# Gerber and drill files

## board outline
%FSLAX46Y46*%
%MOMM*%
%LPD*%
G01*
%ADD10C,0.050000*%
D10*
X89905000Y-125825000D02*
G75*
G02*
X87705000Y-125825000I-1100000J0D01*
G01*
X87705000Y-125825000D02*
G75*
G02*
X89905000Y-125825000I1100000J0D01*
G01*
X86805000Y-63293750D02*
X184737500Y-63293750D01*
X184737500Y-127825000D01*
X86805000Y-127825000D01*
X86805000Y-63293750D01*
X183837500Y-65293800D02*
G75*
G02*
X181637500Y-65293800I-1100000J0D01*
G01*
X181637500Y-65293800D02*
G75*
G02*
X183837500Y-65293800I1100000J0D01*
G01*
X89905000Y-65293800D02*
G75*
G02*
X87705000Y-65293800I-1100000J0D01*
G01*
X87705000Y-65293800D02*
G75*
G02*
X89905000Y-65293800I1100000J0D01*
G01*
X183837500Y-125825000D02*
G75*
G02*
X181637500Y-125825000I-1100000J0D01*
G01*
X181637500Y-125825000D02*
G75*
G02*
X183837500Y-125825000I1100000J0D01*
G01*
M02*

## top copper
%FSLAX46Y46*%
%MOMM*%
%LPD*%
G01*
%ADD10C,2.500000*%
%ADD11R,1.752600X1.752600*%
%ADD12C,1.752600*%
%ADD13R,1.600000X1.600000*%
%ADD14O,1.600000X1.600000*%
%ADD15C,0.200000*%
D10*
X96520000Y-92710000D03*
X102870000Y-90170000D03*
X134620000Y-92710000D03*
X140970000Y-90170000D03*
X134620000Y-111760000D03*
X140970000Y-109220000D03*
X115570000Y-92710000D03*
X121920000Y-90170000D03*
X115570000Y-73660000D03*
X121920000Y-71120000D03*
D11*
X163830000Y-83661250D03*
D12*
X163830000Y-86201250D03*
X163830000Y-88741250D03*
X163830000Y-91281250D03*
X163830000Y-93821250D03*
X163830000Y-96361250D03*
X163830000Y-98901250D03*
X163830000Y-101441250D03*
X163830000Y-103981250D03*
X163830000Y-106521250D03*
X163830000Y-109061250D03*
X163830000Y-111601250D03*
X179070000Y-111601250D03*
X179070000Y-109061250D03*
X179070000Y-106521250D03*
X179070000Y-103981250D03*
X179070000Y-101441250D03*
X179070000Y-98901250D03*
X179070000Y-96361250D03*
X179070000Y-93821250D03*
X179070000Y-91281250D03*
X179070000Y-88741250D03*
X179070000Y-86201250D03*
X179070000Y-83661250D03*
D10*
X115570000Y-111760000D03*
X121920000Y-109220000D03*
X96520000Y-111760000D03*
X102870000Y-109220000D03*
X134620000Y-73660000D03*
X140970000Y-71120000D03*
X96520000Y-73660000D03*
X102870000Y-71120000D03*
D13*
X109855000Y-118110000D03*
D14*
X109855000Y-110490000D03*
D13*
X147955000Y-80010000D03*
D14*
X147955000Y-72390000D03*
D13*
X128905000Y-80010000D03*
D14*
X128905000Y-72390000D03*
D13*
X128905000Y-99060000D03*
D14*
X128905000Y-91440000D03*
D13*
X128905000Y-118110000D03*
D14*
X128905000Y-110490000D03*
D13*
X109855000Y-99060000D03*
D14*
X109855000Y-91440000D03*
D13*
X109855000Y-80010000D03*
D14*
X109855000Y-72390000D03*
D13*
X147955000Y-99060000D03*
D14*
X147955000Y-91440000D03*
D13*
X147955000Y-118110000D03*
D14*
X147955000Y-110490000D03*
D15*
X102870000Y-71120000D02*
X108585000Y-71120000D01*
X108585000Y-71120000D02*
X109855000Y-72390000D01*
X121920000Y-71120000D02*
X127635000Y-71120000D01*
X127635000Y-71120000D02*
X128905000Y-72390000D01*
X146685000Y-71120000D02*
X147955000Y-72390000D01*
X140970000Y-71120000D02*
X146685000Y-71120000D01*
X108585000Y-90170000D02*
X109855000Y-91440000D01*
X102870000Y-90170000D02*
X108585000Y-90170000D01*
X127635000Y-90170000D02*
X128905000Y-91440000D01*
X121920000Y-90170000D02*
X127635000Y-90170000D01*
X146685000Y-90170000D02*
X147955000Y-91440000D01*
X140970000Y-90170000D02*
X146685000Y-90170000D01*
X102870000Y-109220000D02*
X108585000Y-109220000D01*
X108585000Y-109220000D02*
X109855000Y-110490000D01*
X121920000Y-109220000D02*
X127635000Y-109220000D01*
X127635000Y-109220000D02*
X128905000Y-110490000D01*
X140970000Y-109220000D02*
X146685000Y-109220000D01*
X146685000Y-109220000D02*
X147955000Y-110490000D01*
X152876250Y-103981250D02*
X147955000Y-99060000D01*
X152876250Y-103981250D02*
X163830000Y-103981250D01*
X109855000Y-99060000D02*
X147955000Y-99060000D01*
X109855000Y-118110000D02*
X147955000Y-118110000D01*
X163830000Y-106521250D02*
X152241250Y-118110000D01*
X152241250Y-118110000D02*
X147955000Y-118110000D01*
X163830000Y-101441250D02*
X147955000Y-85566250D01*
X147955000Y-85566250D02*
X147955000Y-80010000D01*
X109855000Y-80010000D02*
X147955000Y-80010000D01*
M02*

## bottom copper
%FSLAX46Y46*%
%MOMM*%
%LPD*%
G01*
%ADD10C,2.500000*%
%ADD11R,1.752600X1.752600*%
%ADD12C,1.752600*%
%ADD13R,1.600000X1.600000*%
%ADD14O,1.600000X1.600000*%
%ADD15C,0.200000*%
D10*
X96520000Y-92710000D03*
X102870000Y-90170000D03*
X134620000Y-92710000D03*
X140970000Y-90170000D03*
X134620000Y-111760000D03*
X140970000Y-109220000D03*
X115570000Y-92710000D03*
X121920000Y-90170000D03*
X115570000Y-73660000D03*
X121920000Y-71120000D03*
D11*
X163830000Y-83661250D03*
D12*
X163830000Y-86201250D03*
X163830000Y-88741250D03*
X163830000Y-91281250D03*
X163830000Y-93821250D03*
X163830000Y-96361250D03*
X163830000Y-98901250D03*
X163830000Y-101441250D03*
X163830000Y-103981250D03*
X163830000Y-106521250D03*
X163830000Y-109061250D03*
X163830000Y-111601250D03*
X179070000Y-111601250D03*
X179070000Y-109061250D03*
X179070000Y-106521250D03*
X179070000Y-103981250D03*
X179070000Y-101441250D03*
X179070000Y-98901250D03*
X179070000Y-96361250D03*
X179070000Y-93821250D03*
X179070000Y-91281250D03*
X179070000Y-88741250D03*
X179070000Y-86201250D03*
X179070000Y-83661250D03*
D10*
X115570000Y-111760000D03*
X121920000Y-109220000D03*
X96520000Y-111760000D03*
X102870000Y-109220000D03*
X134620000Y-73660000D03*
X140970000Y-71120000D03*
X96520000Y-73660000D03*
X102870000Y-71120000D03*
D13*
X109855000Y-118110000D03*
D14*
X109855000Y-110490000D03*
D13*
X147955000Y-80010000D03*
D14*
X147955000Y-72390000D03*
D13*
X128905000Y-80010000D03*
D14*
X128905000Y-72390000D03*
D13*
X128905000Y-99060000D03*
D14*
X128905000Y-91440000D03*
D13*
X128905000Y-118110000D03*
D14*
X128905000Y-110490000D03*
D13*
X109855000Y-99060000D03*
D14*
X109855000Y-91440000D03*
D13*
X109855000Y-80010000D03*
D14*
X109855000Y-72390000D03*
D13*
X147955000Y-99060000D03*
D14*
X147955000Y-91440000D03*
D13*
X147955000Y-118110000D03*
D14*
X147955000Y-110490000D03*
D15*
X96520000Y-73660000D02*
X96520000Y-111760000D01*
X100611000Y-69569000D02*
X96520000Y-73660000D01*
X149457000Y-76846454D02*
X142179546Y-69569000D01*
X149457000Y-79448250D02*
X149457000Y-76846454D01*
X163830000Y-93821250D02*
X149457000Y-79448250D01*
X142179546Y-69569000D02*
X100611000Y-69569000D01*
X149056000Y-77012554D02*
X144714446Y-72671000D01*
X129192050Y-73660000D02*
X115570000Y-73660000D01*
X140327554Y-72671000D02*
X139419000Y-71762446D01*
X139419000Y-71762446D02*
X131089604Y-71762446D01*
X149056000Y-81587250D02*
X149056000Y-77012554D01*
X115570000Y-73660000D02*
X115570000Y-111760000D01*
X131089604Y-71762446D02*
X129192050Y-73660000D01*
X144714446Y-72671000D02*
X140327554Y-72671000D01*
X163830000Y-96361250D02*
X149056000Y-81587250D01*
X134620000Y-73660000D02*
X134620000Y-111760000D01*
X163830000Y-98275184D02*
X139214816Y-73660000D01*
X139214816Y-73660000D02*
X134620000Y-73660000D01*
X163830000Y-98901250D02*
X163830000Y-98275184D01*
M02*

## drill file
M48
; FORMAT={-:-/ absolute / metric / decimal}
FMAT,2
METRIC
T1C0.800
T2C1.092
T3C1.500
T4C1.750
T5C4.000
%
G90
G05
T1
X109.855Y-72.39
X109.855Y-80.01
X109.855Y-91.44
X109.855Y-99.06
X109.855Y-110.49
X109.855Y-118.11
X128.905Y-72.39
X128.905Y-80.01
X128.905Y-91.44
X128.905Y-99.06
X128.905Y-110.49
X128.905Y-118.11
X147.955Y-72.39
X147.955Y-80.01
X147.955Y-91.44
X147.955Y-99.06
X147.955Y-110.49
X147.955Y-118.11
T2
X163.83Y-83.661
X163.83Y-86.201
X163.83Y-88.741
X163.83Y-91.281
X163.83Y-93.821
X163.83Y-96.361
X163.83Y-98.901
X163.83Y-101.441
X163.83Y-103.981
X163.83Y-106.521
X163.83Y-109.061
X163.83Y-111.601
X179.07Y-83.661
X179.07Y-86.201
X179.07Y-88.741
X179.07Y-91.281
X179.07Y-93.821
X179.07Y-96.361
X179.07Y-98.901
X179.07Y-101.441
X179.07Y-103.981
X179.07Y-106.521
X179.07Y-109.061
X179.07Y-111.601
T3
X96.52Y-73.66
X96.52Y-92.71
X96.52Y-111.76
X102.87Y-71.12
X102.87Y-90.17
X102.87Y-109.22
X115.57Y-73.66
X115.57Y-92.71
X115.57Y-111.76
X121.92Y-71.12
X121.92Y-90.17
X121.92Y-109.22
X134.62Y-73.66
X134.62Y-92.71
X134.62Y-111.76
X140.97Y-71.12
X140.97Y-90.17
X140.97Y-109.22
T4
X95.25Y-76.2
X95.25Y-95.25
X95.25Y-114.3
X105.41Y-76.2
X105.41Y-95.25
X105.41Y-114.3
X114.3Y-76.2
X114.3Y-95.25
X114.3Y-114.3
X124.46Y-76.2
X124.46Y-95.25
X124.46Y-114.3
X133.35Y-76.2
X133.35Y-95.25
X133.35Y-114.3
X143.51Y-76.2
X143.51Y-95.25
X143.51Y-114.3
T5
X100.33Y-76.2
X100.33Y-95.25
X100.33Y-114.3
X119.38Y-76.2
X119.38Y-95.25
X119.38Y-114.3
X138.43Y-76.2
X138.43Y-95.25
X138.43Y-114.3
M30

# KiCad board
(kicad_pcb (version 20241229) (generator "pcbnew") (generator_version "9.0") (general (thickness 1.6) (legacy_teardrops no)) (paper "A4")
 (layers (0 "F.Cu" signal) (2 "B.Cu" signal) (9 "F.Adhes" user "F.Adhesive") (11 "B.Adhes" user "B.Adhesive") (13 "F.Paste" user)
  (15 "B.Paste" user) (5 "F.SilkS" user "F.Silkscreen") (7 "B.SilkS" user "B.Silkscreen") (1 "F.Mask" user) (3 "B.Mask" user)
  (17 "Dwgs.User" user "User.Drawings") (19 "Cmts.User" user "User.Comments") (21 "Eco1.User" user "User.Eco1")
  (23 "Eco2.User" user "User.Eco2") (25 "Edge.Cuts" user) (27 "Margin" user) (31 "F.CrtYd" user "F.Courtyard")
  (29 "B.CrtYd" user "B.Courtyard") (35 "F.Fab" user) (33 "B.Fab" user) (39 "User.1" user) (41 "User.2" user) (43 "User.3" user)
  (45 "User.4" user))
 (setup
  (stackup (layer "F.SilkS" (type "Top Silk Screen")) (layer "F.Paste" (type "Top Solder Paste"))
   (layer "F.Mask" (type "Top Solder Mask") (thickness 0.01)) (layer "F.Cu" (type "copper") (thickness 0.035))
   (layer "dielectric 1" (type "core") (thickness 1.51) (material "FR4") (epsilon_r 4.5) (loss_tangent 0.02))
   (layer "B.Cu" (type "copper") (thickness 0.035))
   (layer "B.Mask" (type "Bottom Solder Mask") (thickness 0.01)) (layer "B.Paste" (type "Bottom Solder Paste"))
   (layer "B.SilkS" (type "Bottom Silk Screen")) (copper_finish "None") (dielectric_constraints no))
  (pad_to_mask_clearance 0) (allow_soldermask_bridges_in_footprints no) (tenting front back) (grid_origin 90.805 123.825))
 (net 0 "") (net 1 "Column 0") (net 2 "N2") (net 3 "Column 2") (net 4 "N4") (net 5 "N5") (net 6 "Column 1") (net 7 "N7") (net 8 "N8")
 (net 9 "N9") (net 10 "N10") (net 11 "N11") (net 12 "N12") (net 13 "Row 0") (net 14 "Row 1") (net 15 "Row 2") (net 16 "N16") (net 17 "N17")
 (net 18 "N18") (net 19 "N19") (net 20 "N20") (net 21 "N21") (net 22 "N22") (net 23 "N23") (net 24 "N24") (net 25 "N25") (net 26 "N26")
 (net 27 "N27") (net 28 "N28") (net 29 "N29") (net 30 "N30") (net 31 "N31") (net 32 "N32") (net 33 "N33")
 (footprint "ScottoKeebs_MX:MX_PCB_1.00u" (layer "F.Cu") (at 100.33 95.25)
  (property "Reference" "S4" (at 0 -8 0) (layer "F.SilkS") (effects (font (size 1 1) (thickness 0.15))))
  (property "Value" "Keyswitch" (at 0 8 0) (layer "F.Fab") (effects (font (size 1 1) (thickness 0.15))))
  (pad "" np_thru_hole circle (at -5.08 0) (size 1.75 1.75) (drill 1.75) (layers "*.Cu" "*.Mask"))
  (pad "" np_thru_hole circle (at 0 0) (size 4 4) (drill 4) (layers "*.Cu" "*.Mask"))
  (pad "" np_thru_hole circle (at 5.08 0) (size 1.75 1.75) (drill 1.75) (layers "*.Cu" "*.Mask"))
  (pad "1" thru_hole circle (at -3.81 -2.54) (size 2.5 2.5) (drill 1.5) (layers "*.Cu" "*.Mask") (remove_unused_layers no)
   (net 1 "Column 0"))
  (pad "2" thru_hole circle (at 2.54 -5.08) (size 2.5 2.5) (drill 1.5) (layers "*.Cu" "*.Mask") (remove_unused_layers no) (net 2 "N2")))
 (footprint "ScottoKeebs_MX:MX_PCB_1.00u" (layer "F.Cu") (at 138.43 95.25)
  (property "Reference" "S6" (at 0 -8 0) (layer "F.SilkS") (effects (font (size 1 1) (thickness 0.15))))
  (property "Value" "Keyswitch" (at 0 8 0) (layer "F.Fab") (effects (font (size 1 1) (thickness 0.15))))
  (pad "" np_thru_hole circle (at -5.08 0) (size 1.75 1.75) (drill 1.75) (layers "*.Cu" "*.Mask"))
  (pad "" np_thru_hole circle (at 0 0) (size 4 4) (drill 4) (layers "*.Cu" "*.Mask"))
  (pad "" np_thru_hole circle (at 5.08 0) (size 1.75 1.75) (drill 1.75) (layers "*.Cu" "*.Mask"))
  (pad "1" thru_hole circle (at -3.81 -2.54) (size 2.5 2.5) (drill 1.5) (layers "*.Cu" "*.Mask") (remove_unused_layers no)
   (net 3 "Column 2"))
  (pad "2" thru_hole circle (at 2.54 -5.08) (size 2.5 2.5) (drill 1.5) (layers "*.Cu" "*.Mask") (remove_unused_layers no) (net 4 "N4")))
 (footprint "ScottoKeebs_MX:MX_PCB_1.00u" (layer "F.Cu") (at 138.43 114.3)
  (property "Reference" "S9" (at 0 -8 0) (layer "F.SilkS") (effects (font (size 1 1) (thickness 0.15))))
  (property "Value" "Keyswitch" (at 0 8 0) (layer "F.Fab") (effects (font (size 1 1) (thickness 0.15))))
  (pad "" np_thru_hole circle (at -5.08 0) (size 1.75 1.75) (drill 1.75) (layers "*.Cu" "*.Mask"))
  (pad "" np_thru_hole circle (at 0 0) (size 4 4) (drill 4) (layers "*.Cu" "*.Mask"))
  (pad "" np_thru_hole circle (at 5.08 0) (size 1.75 1.75) (drill 1.75) (layers "*.Cu" "*.Mask"))
  (pad "1" thru_hole circle (at -3.81 -2.54) (size 2.5 2.5) (drill 1.5) (layers "*.Cu" "*.Mask") (remove_unused_layers no)
   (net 3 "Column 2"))
  (pad "2" thru_hole circle (at 2.54 -5.08) (size 2.5 2.5) (drill 1.5) (layers "*.Cu" "*.Mask") (remove_unused_layers no) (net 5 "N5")))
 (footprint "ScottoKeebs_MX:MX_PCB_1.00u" (layer "F.Cu") (at 119.38 95.25)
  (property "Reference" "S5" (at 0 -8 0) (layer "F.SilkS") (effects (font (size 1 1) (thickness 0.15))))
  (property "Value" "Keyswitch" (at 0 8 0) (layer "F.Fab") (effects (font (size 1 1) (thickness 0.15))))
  (pad "" np_thru_hole circle (at -5.08 0) (size 1.75 1.75) (drill 1.75) (layers "*.Cu" "*.Mask"))
  (pad "" np_thru_hole circle (at 0 0) (size 4 4) (drill 4) (layers "*.Cu" "*.Mask"))
  (pad "" np_thru_hole circle (at 5.08 0) (size 1.75 1.75) (drill 1.75) (layers "*.Cu" "*.Mask"))
  (pad "1" thru_hole circle (at -3.81 -2.54) (size 2.5 2.5) (drill 1.5) (layers "*.Cu" "*.Mask") (remove_unused_layers no)
   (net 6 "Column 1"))
  (pad "2" thru_hole circle (at 2.54 -5.08) (size 2.5 2.5) (drill 1.5) (layers "*.Cu" "*.Mask") (remove_unused_layers no) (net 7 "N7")))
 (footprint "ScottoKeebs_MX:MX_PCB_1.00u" (layer "F.Cu") (at 119.38 76.2)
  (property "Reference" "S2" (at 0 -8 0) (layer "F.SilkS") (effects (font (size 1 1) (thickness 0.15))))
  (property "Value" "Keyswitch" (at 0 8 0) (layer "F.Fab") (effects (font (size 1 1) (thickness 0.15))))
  (pad "" np_thru_hole circle (at -5.08 0) (size 1.75 1.75) (drill 1.75) (layers "*.Cu" "*.Mask"))
  (pad "" np_thru_hole circle (at 0 0) (size 4 4) (drill 4) (layers "*.Cu" "*.Mask"))
  (pad "" np_thru_hole circle (at 5.08 0) (size 1.75 1.75) (drill 1.75) (layers "*.Cu" "*.Mask"))
  (pad "1" thru_hole circle (at -3.81 -2.54) (size 2.5 2.5) (drill 1.5) (layers "*.Cu" "*.Mask") (remove_unused_layers no)
   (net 6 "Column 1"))
  (pad "2" thru_hole circle (at 2.54 -5.08) (size 2.5 2.5) (drill 1.5) (layers "*.Cu" "*.Mask") (remove_unused_layers no) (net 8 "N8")))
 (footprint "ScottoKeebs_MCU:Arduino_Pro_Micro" (layer "F.Cu") (at 171.45 97.63125)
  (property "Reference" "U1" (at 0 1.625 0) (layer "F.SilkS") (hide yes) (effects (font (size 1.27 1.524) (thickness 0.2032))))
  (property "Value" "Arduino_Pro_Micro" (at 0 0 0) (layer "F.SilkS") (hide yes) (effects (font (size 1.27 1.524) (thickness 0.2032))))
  (pad "1" thru_hole rect (at -7.62 -13.97 270) (size 1.7526 1.7526) (drill 1.0922) (layers "*.Cu" "*.SilkS" "*.Mask")
   (remove_unused_layers no) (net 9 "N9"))
  (pad "2" thru_hole circle (at -7.62 -11.43 270) (size 1.7526 1.7526) (drill 1.0922) (layers "*.Cu" "*.SilkS" "*.Mask")
   (remove_unused_layers no) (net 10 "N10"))
  (pad "3" thru_hole circle (at -7.62 -8.89 270) (size 1.7526 1.7526) (drill 1.0922) (layers "*.Cu" "*.SilkS" "*.Mask")
   (remove_unused_layers no) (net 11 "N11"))
  (pad "4" thru_hole circle (at -7.62 -6.35 270) (size 1.7526 1.7526) (drill 1.0922) (layers "*.Cu" "*.SilkS" "*.Mask")
   (remove_unused_layers no) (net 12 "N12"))
  (pad "5" thru_hole circle (at -7.62 -3.81 270) (size 1.7526 1.7526) (drill 1.0922) (layers "*.Cu" "*.SilkS" "*.Mask")
   (remove_unused_layers no) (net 1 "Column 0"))
  (pad "6" thru_hole circle (at -7.62 -1.27 270) (size 1.7526 1.7526) (drill 1.0922) (layers "*.Cu" "*.SilkS" "*.Mask")
   (remove_unused_layers no) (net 6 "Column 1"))
  (pad "7" thru_hole circle (at -7.62 1.27 270) (size 1.7526 1.7526) (drill 1.0922) (layers "*.Cu" "*.SilkS" "*.Mask")
   (remove_unused_layers no) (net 3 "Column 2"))
  (pad "8" thru_hole circle (at -7.62 3.81 270) (size 1.7526 1.7526) (drill 1.0922) (layers "*.Cu" "*.SilkS" "*.Mask")
   (remove_unused_layers no) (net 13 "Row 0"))
  (pad "9" thru_hole circle (at -7.62 6.35 270) (size 1.7526 1.7526) (drill 1.0922) (layers "*.Cu" "*.SilkS" "*.Mask")
   (remove_unused_layers no) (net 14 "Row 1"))
  (pad "10" thru_hole circle (at -7.62 8.89 270) (size 1.7526 1.7526) (drill 1.0922) (layers "*.Cu" "*.SilkS" "*.Mask")
   (remove_unused_layers no) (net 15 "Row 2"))
  (pad "11" thru_hole circle (at -7.62 11.43 270) (size 1.7526 1.7526) (drill 1.0922) (layers "*.Cu" "*.SilkS" "*.Mask")
   (remove_unused_layers no) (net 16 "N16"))
  (pad "12" thru_hole circle (at -7.62 13.97 270) (size 1.7526 1.7526) (drill 1.0922) (layers "*.Cu" "*.SilkS" "*.Mask")
   (remove_unused_layers no) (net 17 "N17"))
  (pad "13" thru_hole circle (at 7.62 13.97 270) (size 1.7526 1.7526) (drill 1.0922) (layers "*.Cu" "*.SilkS" "*.Mask")
   (remove_unused_layers no) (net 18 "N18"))
  (pad "14" thru_hole circle (at 7.62 11.43 270) (size 1.7526 1.7526) (drill 1.0922) (layers "*.Cu" "*.SilkS" "*.Mask")
   (remove_unused_layers no) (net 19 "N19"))
  (pad "15" thru_hole circle (at 7.62 8.89 270) (size 1.7526 1.7526) (drill 1.0922) (layers "*.Cu" "*.SilkS" "*.Mask")
   (remove_unused_layers no) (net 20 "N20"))
  (pad "16" thru_hole circle (at 7.62 6.35 270) (size 1.7526 1.7526) (drill 1.0922) (layers "*.Cu" "*.SilkS" "*.Mask")
   (remove_unused_layers no) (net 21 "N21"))
  (pad "17" thru_hole circle (at 7.62 3.81 270) (size 1.7526 1.7526) (drill 1.0922) (layers "*.Cu" "*.SilkS" "*.Mask")
   (remove_unused_layers no) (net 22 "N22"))
  (pad "18" thru_hole circle (at 7.62 1.27 270) (size 1.7526 1.7526) (drill 1.0922) (layers "*.Cu" "*.SilkS" "*.Mask")
   (remove_unused_layers no) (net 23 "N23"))
  (pad "19" thru_hole circle (at 7.62 -1.27 270) (size 1.7526 1.7526) (drill 1.0922) (layers "*.Cu" "*.SilkS" "*.Mask")
   (remove_unused_layers no) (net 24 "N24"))
  (pad "20" thru_hole circle (at 7.62 -3.81 270) (size 1.7526 1.7526) (drill 1.0922) (layers "*.Cu" "*.SilkS" "*.Mask")
   (remove_unused_layers no) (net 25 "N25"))
  (pad "21" thru_hole circle (at 7.62 -6.35 270) (size 1.7526 1.7526) (drill 1.0922) (layers "*.Cu" "*.SilkS" "*.Mask")
   (remove_unused_layers no) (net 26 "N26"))
  (pad "22" thru_hole circle (at 7.62 -8.89 270) (size 1.7526 1.7526) (drill 1.0922) (layers "*.Cu" "*.SilkS" "*.Mask")
   (remove_unused_layers no) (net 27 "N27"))
  (pad "23" thru_hole circle (at 7.62 -11.43 270) (size 1.7526 1.7526) (drill 1.0922) (layers "*.Cu" "*.SilkS" "*.Mask")
   (remove_unused_layers no) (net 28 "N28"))
  (pad "24" thru_hole circle (at 7.62 -13.97 270) (size 1.7526 1.7526) (drill 1.0922) (layers "*.Cu" "*.SilkS" "*.Mask")
   (remove_unused_layers no) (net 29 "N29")))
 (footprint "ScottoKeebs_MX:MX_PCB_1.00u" (layer "F.Cu") (at 119.38 114.3)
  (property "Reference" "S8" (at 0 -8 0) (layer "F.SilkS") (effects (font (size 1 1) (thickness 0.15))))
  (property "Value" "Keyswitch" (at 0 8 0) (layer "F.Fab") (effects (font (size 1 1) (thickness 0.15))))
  (pad "" np_thru_hole circle (at -5.08 0) (size 1.75 1.75) (drill 1.75) (layers "*.Cu" "*.Mask"))
  (pad "" np_thru_hole circle (at 0 0) (size 4 4) (drill 4) (layers "*.Cu" "*.Mask"))
  (pad "" np_thru_hole circle (at 5.08 0) (size 1.75 1.75) (drill 1.75) (layers "*.Cu" "*.Mask"))
  (pad "1" thru_hole circle (at -3.81 -2.54) (size 2.5 2.5) (drill 1.5) (layers "*.Cu" "*.Mask") (remove_unused_layers no)
   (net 6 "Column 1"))
  (pad "2" thru_hole circle (at 2.54 -5.08) (size 2.5 2.5) (drill 1.5) (layers "*.Cu" "*.Mask") (remove_unused_layers no) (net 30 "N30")))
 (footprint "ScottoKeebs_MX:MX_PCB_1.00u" (layer "F.Cu") (at 100.33 114.3)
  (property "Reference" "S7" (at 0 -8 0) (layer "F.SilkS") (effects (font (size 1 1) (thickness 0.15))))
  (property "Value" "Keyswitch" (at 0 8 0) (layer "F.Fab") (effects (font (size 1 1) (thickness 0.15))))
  (pad "" np_thru_hole circle (at -5.08 0) (size 1.75 1.75) (drill 1.75) (layers "*.Cu" "*.Mask"))
  (pad "" np_thru_hole circle (at 0 0) (size 4 4) (drill 4) (layers "*.Cu" "*.Mask"))
  (pad "" np_thru_hole circle (at 5.08 0) (size 1.75 1.75) (drill 1.75) (layers "*.Cu" "*.Mask"))
  (pad "1" thru_hole circle (at -3.81 -2.54) (size 2.5 2.5) (drill 1.5) (layers "*.Cu" "*.Mask") (remove_unused_layers no)
   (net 1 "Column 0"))
  (pad "2" thru_hole circle (at 2.54 -5.08) (size 2.5 2.5) (drill 1.5) (layers "*.Cu" "*.Mask") (remove_unused_layers no) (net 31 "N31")))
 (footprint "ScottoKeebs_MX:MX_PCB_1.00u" (layer "F.Cu") (at 138.43 76.2)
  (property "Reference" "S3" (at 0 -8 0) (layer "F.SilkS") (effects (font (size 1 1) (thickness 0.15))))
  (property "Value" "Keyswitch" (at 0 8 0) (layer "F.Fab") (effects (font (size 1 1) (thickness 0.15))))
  (pad "" np_thru_hole circle (at -5.08 0) (size 1.75 1.75) (drill 1.75) (layers "*.Cu" "*.Mask"))
  (pad "" np_thru_hole circle (at 0 0) (size 4 4) (drill 4) (layers "*.Cu" "*.Mask"))
  (pad "" np_thru_hole circle (at 5.08 0) (size 1.75 1.75) (drill 1.75) (layers "*.Cu" "*.Mask"))
  (pad "1" thru_hole circle (at -3.81 -2.54) (size 2.5 2.5) (drill 1.5) (layers "*.Cu" "*.Mask") (remove_unused_layers no)
   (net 3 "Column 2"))
  (pad "2" thru_hole circle (at 2.54 -5.08) (size 2.5 2.5) (drill 1.5) (layers "*.Cu" "*.Mask") (remove_unused_layers no) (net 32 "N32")))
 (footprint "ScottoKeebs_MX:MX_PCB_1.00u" (layer "F.Cu") (at 100.33 76.2)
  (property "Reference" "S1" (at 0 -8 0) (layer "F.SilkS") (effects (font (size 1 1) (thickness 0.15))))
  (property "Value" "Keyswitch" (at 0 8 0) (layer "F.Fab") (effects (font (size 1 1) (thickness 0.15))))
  (pad "" np_thru_hole circle (at -5.08 0) (size 1.75 1.75) (drill 1.75) (layers "*.Cu" "*.Mask"))
  (pad "" np_thru_hole circle (at 0 0) (size 4 4) (drill 4) (layers "*.Cu" "*.Mask"))
  (pad "" np_thru_hole circle (at 5.08 0) (size 1.75 1.75) (drill 1.75) (layers "*.Cu" "*.Mask"))
  (pad "1" thru_hole circle (at -3.81 -2.54) (size 2.5 2.5) (drill 1.5) (layers "*.Cu" "*.Mask") (remove_unused_layers no)
   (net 1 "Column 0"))
  (pad "2" thru_hole circle (at 2.54 -5.08) (size 2.5 2.5) (drill 1.5) (layers "*.Cu" "*.Mask") (remove_unused_layers no) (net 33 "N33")))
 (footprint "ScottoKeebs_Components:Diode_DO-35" (layer "B.Cu") (at 109.855 118.11 90)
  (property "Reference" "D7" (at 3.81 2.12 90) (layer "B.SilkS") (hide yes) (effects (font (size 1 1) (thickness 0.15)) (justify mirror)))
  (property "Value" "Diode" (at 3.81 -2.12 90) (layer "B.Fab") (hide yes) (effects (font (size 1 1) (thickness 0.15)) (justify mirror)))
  (pad "1" thru_hole rect (at 0 0 90) (size 1.6 1.6) (drill 0.8) (layers "*.Cu" "*.Mask") (remove_unused_layers no) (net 15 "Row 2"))
  (pad "2" thru_hole oval (at 7.62 0 90) (size 1.6 1.6) (drill 0.8) (layers "*.Cu" "*.Mask") (remove_unused_layers no) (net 31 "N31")))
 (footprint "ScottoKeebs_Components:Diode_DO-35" (layer "B.Cu") (at 147.955 80.01 90)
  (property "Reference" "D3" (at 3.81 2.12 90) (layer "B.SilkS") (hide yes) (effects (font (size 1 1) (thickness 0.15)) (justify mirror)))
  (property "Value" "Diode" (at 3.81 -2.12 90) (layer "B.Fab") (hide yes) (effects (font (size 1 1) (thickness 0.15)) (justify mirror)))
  (pad "1" thru_hole rect (at 0 0 90) (size 1.6 1.6) (drill 0.8) (layers "*.Cu" "*.Mask") (remove_unused_layers no) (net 13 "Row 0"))
  (pad "2" thru_hole oval (at 7.62 0 90) (size 1.6 1.6) (drill 0.8) (layers "*.Cu" "*.Mask") (remove_unused_layers no) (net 32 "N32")))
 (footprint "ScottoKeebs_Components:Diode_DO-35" (layer "B.Cu") (at 128.905 80.01 90)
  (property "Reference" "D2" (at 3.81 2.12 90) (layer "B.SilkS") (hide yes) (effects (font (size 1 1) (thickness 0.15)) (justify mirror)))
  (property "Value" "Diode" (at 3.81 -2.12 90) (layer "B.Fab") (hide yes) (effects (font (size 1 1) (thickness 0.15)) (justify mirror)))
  (pad "1" thru_hole rect (at 0 0 90) (size 1.6 1.6) (drill 0.8) (layers "*.Cu" "*.Mask") (remove_unused_layers no) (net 13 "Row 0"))
  (pad "2" thru_hole oval (at 7.62 0 90) (size 1.6 1.6) (drill 0.8) (layers "*.Cu" "*.Mask") (remove_unused_layers no) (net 8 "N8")))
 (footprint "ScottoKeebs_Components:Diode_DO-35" (layer "B.Cu") (at 128.905 99.06 90)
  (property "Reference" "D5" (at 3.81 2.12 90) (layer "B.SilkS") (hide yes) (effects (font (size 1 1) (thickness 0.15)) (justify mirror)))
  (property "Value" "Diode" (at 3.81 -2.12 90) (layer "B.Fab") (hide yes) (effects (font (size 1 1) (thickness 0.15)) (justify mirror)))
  (pad "1" thru_hole rect (at 0 0 90) (size 1.6 1.6) (drill 0.8) (layers "*.Cu" "*.Mask") (remove_unused_layers no) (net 14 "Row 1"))
  (pad "2" thru_hole oval (at 7.62 0 90) (size 1.6 1.6) (drill 0.8) (layers "*.Cu" "*.Mask") (remove_unused_layers no) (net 7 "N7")))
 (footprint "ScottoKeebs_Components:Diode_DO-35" (layer "B.Cu") (at 128.905 118.11 90)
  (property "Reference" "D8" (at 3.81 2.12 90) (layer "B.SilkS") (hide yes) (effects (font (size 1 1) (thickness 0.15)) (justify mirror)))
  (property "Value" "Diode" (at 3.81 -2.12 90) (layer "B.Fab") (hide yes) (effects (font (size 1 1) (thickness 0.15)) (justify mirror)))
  (pad "1" thru_hole rect (at 0 0 90) (size 1.6 1.6) (drill 0.8) (layers "*.Cu" "*.Mask") (remove_unused_layers no) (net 15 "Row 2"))
  (pad "2" thru_hole oval (at 7.62 0 90) (size 1.6 1.6) (drill 0.8) (layers "*.Cu" "*.Mask") (remove_unused_layers no) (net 30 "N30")))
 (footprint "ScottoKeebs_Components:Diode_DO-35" (layer "B.Cu") (at 109.855 99.06 90)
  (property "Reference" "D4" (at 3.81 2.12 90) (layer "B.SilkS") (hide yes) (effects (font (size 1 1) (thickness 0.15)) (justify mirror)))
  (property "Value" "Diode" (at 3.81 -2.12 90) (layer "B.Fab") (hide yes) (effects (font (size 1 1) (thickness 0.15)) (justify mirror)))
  (pad "1" thru_hole rect (at 0 0 90) (size 1.6 1.6) (drill 0.8) (layers "*.Cu" "*.Mask") (remove_unused_layers no) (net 14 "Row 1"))
  (pad "2" thru_hole oval (at 7.62 0 90) (size 1.6 1.6) (drill 0.8) (layers "*.Cu" "*.Mask") (remove_unused_layers no) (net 2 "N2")))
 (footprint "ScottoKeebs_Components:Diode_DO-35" (layer "B.Cu") (at 109.855 80.01 90)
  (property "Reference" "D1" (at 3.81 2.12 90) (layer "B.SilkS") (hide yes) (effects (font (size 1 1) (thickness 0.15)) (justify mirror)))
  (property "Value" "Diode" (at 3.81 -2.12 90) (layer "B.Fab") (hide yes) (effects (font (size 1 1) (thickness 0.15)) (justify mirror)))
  (pad "1" thru_hole rect (at 0 0 90) (size 1.6 1.6) (drill 0.8) (layers "*.Cu" "*.Mask") (remove_unused_layers no) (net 13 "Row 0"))
  (pad "2" thru_hole oval (at 7.62 0 90) (size 1.6 1.6) (drill 0.8) (layers "*.Cu" "*.Mask") (remove_unused_layers no) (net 33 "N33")))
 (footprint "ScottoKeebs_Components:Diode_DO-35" (layer "B.Cu") (at 147.955 99.06 90)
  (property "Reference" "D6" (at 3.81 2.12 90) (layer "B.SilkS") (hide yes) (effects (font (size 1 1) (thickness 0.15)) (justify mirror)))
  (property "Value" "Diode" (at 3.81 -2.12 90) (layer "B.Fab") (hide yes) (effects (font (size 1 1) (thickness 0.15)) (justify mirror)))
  (pad "1" thru_hole rect (at 0 0 90) (size 1.6 1.6) (drill 0.8) (layers "*.Cu" "*.Mask") (remove_unused_layers no) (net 14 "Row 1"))
  (pad "2" thru_hole oval (at 7.62 0 90) (size 1.6 1.6) (drill 0.8) (layers "*.Cu" "*.Mask") (remove_unused_layers no) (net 4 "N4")))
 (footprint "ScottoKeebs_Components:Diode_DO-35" (layer "B.Cu") (at 147.955 118.11 90)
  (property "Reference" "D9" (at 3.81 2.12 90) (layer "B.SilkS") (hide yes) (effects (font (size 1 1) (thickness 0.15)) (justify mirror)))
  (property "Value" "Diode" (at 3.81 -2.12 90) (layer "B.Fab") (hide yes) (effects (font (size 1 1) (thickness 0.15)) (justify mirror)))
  (pad "1" thru_hole rect (at 0 0 90) (size 1.6 1.6) (drill 0.8) (layers "*.Cu" "*.Mask") (remove_unused_layers no) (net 15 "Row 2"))
  (pad "2" thru_hole oval (at 7.62 0 90) (size 1.6 1.6) (drill 0.8) (layers "*.Cu" "*.Mask") (remove_unused_layers no) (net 5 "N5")))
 (gr_circle (center 88.805 125.825) (end 89.905 125.825) (stroke (width 0.05) (type solid)) (fill no) (layer "Edge.Cuts"))
 (gr_rect (start 86.805 63.29375) (end 184.7375 127.825) (stroke (width 0.05) (type solid)) (fill no) (layer "Edge.Cuts"))
 (gr_circle (center 182.7375 65.2938) (end 183.8375 65.2938) (stroke (width 0.05) (type solid)) (fill no) (layer "Edge.Cuts"))
 (gr_circle (center 88.805 65.2938) (end 89.905 65.2938) (stroke (width 0.05) (type solid)) (fill no) (layer "Edge.Cuts"))
 (gr_circle (center 182.7375 125.825) (end 183.8375 125.825) (stroke (width 0.05) (type solid)) (fill no) (layer "Edge.Cuts"))
 (segment (start 102.87 71.12) (end 108.585 71.12) (width 0.2) (layer "F.Cu") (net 33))
 (segment (start 108.585 71.12) (end 109.855 72.39) (width 0.2) (layer "F.Cu") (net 33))
 (segment (start 96.52 73.66) (end 96.52 111.76) (width 0.2) (layer "B.Cu") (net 1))
 (segment (start 100.611 69.569) (end 96.52 73.66) (width 0.2) (layer "B.Cu") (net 1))
 (segment (start 149.457 76.846454) (end 142.179546 69.569) (width 0.2) (layer "B.Cu") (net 1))
 (segment (start 149.457 79.44825) (end 149.457 76.846454) (width 0.2) (layer "B.Cu") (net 1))
 (segment (start 163.83 93.82125) (end 149.457 79.44825) (width 0.2) (layer "B.Cu") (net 1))
 (segment (start 142.179546 69.569) (end 100.611 69.569) (width 0.2) (layer "B.Cu") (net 1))
 (segment (start 149.056 77.012554) (end 144.714446 72.671) (width 0.2) (layer "B.Cu") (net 6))
 (segment (start 129.19205 73.66) (end 115.57 73.66) (width 0.2) (layer "B.Cu") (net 6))
 (segment (start 140.327554 72.671) (end 139.419 71.762446) (width 0.2) (layer "B.Cu") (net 6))
 (segment (start 139.419 71.762446) (end 131.089604 71.762446) (width 0.2) (layer "B.Cu") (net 6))
 (segment (start 149.056 81.58725) (end 149.056 77.012554) (width 0.2) (layer "B.Cu") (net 6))
 (segment (start 115.57 73.66) (end 115.57 111.76) (width 0.2) (layer "B.Cu") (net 6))
 (segment (start 131.089604 71.762446) (end 129.19205 73.66) (width 0.2) (layer "B.Cu") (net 6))
 (segment (start 144.714446 72.671) (end 140.327554 72.671) (width 0.2) (layer "B.Cu") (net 6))
 (segment (start 163.83 96.36125) (end 149.056 81.58725) (width 0.2) (layer "B.Cu") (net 6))
 (segment (start 121.92 71.12) (end 127.635 71.12) (width 0.2) (layer "F.Cu") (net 8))
 (segment (start 127.635 71.12) (end 128.905 72.39) (width 0.2) (layer "F.Cu") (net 8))
 (segment (start 146.685 71.12) (end 147.955 72.39) (width 0.2) (layer "F.Cu") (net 32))
 (segment (start 140.97 71.12) (end 146.685 71.12) (width 0.2) (layer "F.Cu") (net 32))
 (segment (start 134.62 73.66) (end 134.62 111.76) (width 0.2) (layer "B.Cu") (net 3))
 (segment (start 163.83 98.275184) (end 139.214816 73.66) (width 0.2) (layer "B.Cu") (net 3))
 (segment (start 139.214816 73.66) (end 134.62 73.66) (width 0.2) (layer "B.Cu") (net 3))
 (segment (start 163.83 98.90125) (end 163.83 98.275184) (width 0.2) (layer "B.Cu") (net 3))
 (segment (start 108.585 90.17) (end 109.855 91.44) (width 0.2) (layer "F.Cu") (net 2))
 (segment (start 102.87 90.17) (end 108.585 90.17) (width 0.2) (layer "F.Cu") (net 2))
 (segment (start 127.635 90.17) (end 128.905 91.44) (width 0.2) (layer "F.Cu") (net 7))
 (segment (start 121.92 90.17) (end 127.635 90.17) (width 0.2) (layer "F.Cu") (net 7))
 (segment (start 146.685 90.17) (end 147.955 91.44) (width 0.2) (layer "F.Cu") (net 4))
 (segment (start 140.97 90.17) (end 146.685 90.17) (width 0.2) (layer "F.Cu") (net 4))
 (segment (start 102.87 109.22) (end 108.585 109.22) (width 0.2) (layer "F.Cu") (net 31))
 (segment (start 108.585 109.22) (end 109.855 110.49) (width 0.2) (layer "F.Cu") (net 31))
 (segment (start 121.92 109.22) (end 127.635 109.22) (width 0.2) (layer "F.Cu") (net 30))
 (segment (start 127.635 109.22) (end 128.905 110.49) (width 0.2) (layer "F.Cu") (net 30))
 (segment (start 140.97 109.22) (end 146.685 109.22) (width 0.2) (layer "F.Cu") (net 5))
 (segment (start 146.685 109.22) (end 147.955 110.49) (width 0.2) (layer "F.Cu") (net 5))
 (segment (start 152.87625 103.98125) (end 147.955 99.06) (width 0.2) (layer "F.Cu") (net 14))
 (segment (start 152.87625 103.98125) (end 163.83 103.98125) (width 0.2) (layer "F.Cu") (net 14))
 (segment (start 109.855 99.06) (end 147.955 99.06) (width 0.2) (layer "F.Cu") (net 14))
 (segment (start 109.855 118.11) (end 147.955 118.11) (width 0.2) (layer "F.Cu") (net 15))
 (segment (start 163.83 106.52125) (end 152.24125 118.11) (width 0.2) (layer "F.Cu") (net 15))
 (segment (start 152.24125 118.11) (end 147.955 118.11) (width 0.2) (layer "F.Cu") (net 15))
 (segment (start 163.83 101.44125) (end 147.955 85.56625) (width 0.2) (layer "F.Cu") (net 13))
 (segment (start 147.955 85.56625) (end 147.955 80.01) (width 0.2) (layer "F.Cu") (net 13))
 (segment (start 109.855 80.01) (end 147.955 80.01) (width 0.2) (layer "F.Cu") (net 13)))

